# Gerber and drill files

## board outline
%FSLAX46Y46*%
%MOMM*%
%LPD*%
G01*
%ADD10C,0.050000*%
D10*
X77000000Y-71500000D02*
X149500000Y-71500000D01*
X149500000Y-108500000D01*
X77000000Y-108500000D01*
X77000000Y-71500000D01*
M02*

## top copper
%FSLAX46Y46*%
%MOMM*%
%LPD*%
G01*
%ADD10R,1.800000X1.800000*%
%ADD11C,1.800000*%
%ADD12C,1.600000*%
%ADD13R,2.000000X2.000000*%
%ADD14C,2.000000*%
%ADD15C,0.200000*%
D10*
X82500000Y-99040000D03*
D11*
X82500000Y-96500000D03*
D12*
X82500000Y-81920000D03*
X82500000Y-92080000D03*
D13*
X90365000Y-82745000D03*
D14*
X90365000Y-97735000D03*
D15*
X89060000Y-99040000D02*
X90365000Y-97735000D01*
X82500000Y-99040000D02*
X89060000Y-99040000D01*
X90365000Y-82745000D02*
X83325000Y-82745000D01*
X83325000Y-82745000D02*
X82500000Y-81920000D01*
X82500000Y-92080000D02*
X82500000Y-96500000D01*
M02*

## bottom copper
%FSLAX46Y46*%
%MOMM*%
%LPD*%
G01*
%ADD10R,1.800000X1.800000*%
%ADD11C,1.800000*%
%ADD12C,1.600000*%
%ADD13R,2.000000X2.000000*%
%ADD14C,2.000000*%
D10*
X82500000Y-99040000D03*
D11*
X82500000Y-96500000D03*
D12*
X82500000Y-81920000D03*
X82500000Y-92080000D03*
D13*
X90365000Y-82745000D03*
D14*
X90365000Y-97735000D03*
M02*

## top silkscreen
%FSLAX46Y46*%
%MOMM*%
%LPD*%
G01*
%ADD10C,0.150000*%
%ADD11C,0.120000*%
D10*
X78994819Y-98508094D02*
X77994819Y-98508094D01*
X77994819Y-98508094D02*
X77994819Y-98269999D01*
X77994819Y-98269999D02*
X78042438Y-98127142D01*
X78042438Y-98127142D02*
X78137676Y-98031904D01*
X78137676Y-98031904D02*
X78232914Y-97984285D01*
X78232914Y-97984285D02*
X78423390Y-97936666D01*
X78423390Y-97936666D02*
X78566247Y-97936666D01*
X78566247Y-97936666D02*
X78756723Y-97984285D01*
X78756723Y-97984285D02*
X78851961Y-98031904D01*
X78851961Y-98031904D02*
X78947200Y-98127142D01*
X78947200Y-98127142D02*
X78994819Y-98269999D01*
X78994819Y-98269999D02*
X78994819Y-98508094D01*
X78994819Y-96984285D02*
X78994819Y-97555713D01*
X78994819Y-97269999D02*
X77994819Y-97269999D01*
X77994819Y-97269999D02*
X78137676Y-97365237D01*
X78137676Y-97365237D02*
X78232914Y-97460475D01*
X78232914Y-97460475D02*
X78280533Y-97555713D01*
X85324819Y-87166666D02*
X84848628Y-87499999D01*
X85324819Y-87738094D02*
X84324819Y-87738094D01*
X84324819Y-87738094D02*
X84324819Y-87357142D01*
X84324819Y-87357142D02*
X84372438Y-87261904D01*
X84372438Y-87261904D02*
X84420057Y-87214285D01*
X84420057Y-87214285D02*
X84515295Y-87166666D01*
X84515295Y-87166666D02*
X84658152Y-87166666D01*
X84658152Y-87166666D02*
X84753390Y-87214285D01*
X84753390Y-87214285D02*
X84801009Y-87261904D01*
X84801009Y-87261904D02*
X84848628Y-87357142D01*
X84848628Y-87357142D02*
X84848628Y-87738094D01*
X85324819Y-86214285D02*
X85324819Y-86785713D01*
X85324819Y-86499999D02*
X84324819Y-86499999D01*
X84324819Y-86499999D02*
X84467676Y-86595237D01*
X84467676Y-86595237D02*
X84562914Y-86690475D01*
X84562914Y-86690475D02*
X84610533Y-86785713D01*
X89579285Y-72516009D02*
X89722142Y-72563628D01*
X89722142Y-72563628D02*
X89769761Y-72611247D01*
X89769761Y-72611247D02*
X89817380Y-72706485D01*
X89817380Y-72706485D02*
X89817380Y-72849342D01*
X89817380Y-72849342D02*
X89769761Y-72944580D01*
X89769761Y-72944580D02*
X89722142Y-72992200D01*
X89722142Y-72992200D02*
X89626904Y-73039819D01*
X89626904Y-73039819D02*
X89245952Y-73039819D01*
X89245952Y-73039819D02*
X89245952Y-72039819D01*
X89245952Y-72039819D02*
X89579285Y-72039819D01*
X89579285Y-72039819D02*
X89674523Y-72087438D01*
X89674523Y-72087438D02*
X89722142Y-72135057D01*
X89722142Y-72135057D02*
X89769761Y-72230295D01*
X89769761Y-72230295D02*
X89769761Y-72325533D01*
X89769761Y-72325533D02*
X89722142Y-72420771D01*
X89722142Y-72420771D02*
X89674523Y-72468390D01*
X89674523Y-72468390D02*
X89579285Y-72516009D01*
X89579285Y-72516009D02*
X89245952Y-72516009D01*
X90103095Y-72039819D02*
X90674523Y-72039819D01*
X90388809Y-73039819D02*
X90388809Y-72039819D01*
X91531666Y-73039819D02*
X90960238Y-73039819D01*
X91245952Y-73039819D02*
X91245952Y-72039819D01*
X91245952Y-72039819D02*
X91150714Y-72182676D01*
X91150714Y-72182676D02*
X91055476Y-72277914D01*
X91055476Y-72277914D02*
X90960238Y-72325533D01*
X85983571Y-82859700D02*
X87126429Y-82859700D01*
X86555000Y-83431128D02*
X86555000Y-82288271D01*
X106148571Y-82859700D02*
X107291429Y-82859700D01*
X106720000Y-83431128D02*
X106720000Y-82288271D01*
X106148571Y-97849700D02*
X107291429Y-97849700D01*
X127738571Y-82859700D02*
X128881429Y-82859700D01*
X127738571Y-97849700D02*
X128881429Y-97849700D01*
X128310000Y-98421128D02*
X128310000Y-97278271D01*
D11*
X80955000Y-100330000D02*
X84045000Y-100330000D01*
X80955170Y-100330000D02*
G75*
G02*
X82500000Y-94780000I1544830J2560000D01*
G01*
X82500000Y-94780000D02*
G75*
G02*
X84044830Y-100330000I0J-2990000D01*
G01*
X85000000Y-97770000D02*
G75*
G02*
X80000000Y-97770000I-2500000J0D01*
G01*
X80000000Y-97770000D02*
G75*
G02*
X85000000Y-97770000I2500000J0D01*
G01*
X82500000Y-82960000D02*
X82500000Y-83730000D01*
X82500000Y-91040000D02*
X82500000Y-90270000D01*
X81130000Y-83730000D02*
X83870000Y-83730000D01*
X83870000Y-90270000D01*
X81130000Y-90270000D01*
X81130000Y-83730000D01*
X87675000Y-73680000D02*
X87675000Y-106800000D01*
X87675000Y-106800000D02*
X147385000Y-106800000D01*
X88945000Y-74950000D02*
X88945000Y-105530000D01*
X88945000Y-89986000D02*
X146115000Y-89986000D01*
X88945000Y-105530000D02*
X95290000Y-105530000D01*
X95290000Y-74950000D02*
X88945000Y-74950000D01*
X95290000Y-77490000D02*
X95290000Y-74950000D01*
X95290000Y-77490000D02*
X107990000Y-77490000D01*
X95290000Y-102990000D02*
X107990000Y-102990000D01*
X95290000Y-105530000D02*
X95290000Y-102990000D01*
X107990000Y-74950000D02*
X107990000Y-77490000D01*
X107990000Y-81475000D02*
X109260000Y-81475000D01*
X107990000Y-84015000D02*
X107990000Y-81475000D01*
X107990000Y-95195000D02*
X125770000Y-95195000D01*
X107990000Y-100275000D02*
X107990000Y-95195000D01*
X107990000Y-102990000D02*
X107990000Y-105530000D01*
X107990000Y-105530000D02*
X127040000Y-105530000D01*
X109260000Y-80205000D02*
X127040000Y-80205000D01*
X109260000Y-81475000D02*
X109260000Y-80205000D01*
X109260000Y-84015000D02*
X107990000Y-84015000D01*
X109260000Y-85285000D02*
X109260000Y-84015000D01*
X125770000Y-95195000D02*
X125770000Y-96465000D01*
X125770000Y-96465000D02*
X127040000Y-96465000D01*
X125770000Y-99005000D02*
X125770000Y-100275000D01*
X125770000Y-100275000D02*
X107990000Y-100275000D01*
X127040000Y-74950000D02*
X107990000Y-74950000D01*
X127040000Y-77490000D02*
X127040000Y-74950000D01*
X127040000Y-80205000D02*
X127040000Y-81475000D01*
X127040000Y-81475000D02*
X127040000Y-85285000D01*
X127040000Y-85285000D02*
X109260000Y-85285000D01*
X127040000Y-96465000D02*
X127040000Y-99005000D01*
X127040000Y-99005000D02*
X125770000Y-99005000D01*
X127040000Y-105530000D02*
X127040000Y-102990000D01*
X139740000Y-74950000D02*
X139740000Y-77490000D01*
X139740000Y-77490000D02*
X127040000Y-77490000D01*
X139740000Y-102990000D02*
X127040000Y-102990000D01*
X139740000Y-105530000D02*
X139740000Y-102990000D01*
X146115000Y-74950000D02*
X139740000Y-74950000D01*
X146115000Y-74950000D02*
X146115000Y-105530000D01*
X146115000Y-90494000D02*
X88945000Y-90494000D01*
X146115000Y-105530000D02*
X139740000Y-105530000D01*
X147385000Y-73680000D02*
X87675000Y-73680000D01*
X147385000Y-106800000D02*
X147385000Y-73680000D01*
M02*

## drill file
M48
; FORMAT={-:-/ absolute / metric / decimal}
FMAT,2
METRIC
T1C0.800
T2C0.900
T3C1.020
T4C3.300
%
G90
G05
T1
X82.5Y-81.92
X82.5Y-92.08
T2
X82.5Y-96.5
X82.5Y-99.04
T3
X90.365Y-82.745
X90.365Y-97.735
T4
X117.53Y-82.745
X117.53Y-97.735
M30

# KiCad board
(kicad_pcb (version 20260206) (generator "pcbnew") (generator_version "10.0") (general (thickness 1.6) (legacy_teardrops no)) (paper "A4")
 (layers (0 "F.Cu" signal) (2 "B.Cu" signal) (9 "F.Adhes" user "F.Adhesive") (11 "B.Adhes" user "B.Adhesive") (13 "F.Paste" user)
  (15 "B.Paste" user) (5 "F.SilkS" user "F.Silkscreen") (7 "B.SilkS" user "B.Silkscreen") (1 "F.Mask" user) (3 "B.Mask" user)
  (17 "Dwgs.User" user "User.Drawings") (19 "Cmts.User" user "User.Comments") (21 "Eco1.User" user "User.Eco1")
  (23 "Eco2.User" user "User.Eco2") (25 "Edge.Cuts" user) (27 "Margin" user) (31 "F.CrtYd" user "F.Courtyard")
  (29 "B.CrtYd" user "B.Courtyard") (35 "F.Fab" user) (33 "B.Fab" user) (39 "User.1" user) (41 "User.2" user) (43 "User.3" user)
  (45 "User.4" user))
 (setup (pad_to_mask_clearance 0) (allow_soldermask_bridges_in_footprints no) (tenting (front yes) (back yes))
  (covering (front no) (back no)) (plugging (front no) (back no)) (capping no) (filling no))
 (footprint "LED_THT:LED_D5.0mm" (layer "F.Cu") (at 82.5 99.04 90)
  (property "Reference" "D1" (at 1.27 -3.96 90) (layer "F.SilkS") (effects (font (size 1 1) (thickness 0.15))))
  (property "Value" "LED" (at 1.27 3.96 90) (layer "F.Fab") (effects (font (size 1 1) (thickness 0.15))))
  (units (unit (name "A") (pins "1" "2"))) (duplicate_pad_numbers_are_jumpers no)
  (fp_line (start -1.29 -1.545) (end -1.29 1.545) (stroke (width 0.12) (type solid)) (layer "F.SilkS"))
  (fp_arc (start -1.29 -1.54483) (mid 2.071779 -2.880495) (end 4.26 0) (stroke (width 0.12) (type solid)) (layer "F.SilkS"))
  (fp_arc (start 4.26 0) (mid 2.071779 2.880495) (end -1.29 1.54483) (stroke (width 0.12) (type solid)) (layer "F.SilkS"))
  (fp_circle (center 1.27 0) (end 3.77 0) (stroke (width 0.12) (type solid)) (fill no) (layer "F.SilkS"))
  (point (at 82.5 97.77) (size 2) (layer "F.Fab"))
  (pad "1" thru_hole rect (at 0 0 90) (size 1.8 1.8) (drill 0.9) (layers "*.Cu" "*.Mask") (remove_unused_layers no) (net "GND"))
  (pad "2" thru_hole circle (at 2.54 0 90) (size 1.8 1.8) (drill 0.9) (layers "*.Cu" "*.Mask") (remove_unused_layers no) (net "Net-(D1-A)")))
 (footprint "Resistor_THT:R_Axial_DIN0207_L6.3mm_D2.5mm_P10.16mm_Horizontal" (layer "F.Cu") (at 82.5 81.92 -90)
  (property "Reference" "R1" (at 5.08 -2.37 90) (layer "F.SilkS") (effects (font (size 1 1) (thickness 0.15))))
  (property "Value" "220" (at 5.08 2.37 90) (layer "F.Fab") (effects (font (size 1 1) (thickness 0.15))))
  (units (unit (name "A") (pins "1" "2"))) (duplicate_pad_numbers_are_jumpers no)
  (fp_line (start 1.04 0) (end 1.81 0) (stroke (width 0.12) (type solid)) (layer "F.SilkS"))
  (fp_line (start 9.12 0) (end 8.35 0) (stroke (width 0.12) (type solid)) (layer "F.SilkS"))
  (fp_rect (start 1.81 -1.37) (end 8.35 1.37) (stroke (width 0.12) (type solid)) (fill no) (layer "F.SilkS"))
  (pad "1" thru_hole circle (at 0 0 270) (size 1.6 1.6) (drill 0.8) (layers "*.Cu" "*.Mask") (remove_unused_layers no) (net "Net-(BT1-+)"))
  (pad "2" thru_hole circle (at 10.16 0 270) (size 1.6 1.6) (drill 0.8) (layers "*.Cu" "*.Mask") (remove_unused_layers no)
   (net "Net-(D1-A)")))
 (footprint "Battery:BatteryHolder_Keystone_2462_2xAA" (layer "F.Cu") (at 90.365 82.745)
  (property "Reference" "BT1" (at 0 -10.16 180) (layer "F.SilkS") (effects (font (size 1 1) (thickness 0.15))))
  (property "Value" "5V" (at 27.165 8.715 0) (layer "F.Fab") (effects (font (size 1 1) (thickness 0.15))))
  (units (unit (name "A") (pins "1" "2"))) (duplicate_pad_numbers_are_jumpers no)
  (fp_line (start -2.69 -9.065) (end -2.69 24.055) (stroke (width 0.12) (type solid)) (layer "F.SilkS"))
  (fp_line (start -2.69 24.055) (end 57.02 24.055) (stroke (width 0.12) (type solid)) (layer "F.SilkS"))
  (fp_line (start -1.42 -7.795) (end -1.42 22.785) (stroke (width 0.12) (type solid)) (layer "F.SilkS"))
  (fp_line (start -1.42 7.241) (end 55.75 7.241) (stroke (width 0.12) (type solid)) (layer "F.SilkS"))
  (fp_line (start -1.42 22.785) (end 4.925 22.785) (stroke (width 0.12) (type solid)) (layer "F.SilkS"))
  (fp_line (start 4.925 -7.795) (end -1.42 -7.795) (stroke (width 0.12) (type solid)) (layer "F.SilkS"))
  (fp_line (start 4.925 -5.255) (end 4.925 -7.795) (stroke (width 0.12) (type solid)) (layer "F.SilkS"))
  (fp_line (start 4.925 -5.255) (end 17.625 -5.255) (stroke (width 0.12) (type solid)) (layer "F.SilkS"))
  (fp_line (start 4.925 20.245) (end 17.625 20.245) (stroke (width 0.12) (type solid)) (layer "F.SilkS"))
  (fp_line (start 4.925 22.785) (end 4.925 20.245) (stroke (width 0.12) (type solid)) (layer "F.SilkS"))
  (fp_line (start 17.625 -7.795) (end 17.625 -5.255) (stroke (width 0.12) (type solid)) (layer "F.SilkS"))
  (fp_line (start 17.625 -1.27) (end 18.895 -1.27) (stroke (width 0.12) (type solid)) (layer "F.SilkS"))
  (fp_line (start 17.625 1.27) (end 17.625 -1.27) (stroke (width 0.12) (type solid)) (layer "F.SilkS"))
  (fp_line (start 17.625 12.45) (end 35.405 12.45) (stroke (width 0.12) (type solid)) (layer "F.SilkS"))
  (fp_line (start 17.625 17.53) (end 17.625 12.45) (stroke (width 0.12) (type solid)) (layer "F.SilkS"))
  (fp_line (start 17.625 20.245) (end 17.625 22.785) (stroke (width 0.12) (type solid)) (layer "F.SilkS"))
  (fp_line (start 17.625 22.785) (end 36.675 22.785) (stroke (width 0.12) (type solid)) (layer "F.SilkS"))
  (fp_line (start 18.895 -2.54) (end 36.675 -2.54) (stroke (width 0.12) (type solid)) (layer "F.SilkS"))
  (fp_line (start 18.895 -1.27) (end 18.895 -2.54) (stroke (width 0.12) (type solid)) (layer "F.SilkS"))
  (fp_line (start 18.895 1.27) (end 17.625 1.27) (stroke (width 0.12) (type solid)) (layer "F.SilkS"))
  (fp_line (start 18.895 2.54) (end 18.895 1.27) (stroke (width 0.12) (type solid)) (layer "F.SilkS"))
  (fp_line (start 35.405 12.45) (end 35.405 13.72) (stroke (width 0.12) (type solid)) (layer "F.SilkS"))
  (fp_line (start 35.405 13.72) (end 36.675 13.72) (stroke (width 0.12) (type solid)) (layer "F.SilkS"))
  (fp_line (start 35.405 16.26) (end 35.405 17.53) (stroke (width 0.12) (type solid)) (layer "F.SilkS"))
  (fp_line (start 35.405 17.53) (end 17.625 17.53) (stroke (width 0.12) (type solid)) (layer "F.SilkS"))
  (fp_line (start 36.675 -7.795) (end 17.625 -7.795) (stroke (width 0.12) (type solid)) (layer "F.SilkS"))
  (fp_line (start 36.675 -5.255) (end 36.675 -7.795) (stroke (width 0.12) (type solid)) (layer "F.SilkS"))
  (fp_line (start 36.675 -2.54) (end 36.675 -1.27) (stroke (width 0.12) (type solid)) (layer "F.SilkS"))
  (fp_line (start 36.675 -1.27) (end 36.675 2.54) (stroke (width 0.12) (type solid)) (layer "F.SilkS"))
  (fp_line (start 36.675 2.54) (end 18.895 2.54) (stroke (width 0.12) (type solid)) (layer "F.SilkS"))
  (fp_line (start 36.675 13.72) (end 36.675 16.26) (stroke (width 0.12) (type solid)) (layer "F.SilkS"))
  (fp_line (start 36.675 16.26) (end 35.405 16.26) (stroke (width 0.12) (type solid)) (layer "F.SilkS"))
  (fp_line (start 36.675 22.785) (end 36.675 20.245) (stroke (width 0.12) (type solid)) (layer "F.SilkS"))
  (fp_line (start 49.375 -7.795) (end 49.375 -5.255) (stroke (width 0.12) (type solid)) (layer "F.SilkS"))
  (fp_line (start 49.375 -5.255) (end 36.675 -5.255) (stroke (width 0.12) (type solid)) (layer "F.SilkS"))
  (fp_line (start 49.375 20.245) (end 36.675 20.245) (stroke (width 0.12) (type solid)) (layer "F.SilkS"))
  (fp_line (start 49.375 22.785) (end 49.375 20.245) (stroke (width 0.12) (type solid)) (layer "F.SilkS"))
  (fp_line (start 55.75 -7.795) (end 49.375 -7.795) (stroke (width 0.12) (type solid)) (layer "F.SilkS"))
  (fp_line (start 55.75 -7.795) (end 55.75 22.785) (stroke (width 0.12) (type solid)) (layer "F.SilkS"))
  (fp_line (start 55.75 7.749) (end -1.42 7.749) (stroke (width 0.12) (type solid)) (layer "F.SilkS"))
  (fp_line (start 55.75 22.785) (end 49.375 22.785) (stroke (width 0.12) (type solid)) (layer "F.SilkS"))
  (fp_line (start 57.02 -9.065) (end -2.69 -9.065) (stroke (width 0.12) (type solid)) (layer "F.SilkS"))
  (fp_line (start 57.02 24.055) (end 57.02 -9.065) (stroke (width 0.12) (type solid)) (layer "F.SilkS"))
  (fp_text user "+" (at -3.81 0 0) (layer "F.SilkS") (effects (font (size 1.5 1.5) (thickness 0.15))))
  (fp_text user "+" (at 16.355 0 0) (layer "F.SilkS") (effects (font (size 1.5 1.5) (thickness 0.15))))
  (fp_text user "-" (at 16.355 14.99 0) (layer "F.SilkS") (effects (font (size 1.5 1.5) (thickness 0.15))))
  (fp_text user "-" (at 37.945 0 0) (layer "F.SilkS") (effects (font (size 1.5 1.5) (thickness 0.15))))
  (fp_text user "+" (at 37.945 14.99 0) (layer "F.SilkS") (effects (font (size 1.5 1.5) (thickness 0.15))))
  (pad "" np_thru_hole circle (at 27.165 0) (size 3.3 3.3) (drill 3.3) (layers "*.Cu" "*.Mask"))
  (pad "" np_thru_hole circle (at 27.165 14.99) (size 3.3 3.3) (drill 3.3) (layers "*.Cu" "*.Mask"))
  (pad "1" thru_hole rect (at 0 0) (size 2 2) (drill 1.02) (layers "*.Cu" "*.Mask") (remove_unused_layers no) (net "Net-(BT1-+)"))
  (pad "2" thru_hole circle (at 0 14.99) (size 2 2) (drill 1.02) (layers "*.Cu" "*.Mask") (remove_unused_layers no) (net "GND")))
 (gr_rect (start 77 71.5) (end 149.5 108.5) (stroke (width 0.05) (type default)) (fill no) (layer "Edge.Cuts"))
 (segment (start 89.06 99.04) (end 90.365 97.735) (width 0.2) (layer "F.Cu") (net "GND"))
 (segment (start 82.5 99.04) (end 89.06 99.04) (width 0.2) (layer "F.Cu") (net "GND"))
 (segment (start 90.365 82.745) (end 83.325 82.745) (width 0.2) (layer "F.Cu") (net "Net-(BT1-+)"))
 (segment (start 83.325 82.745) (end 82.5 81.92) (width 0.2) (layer "F.Cu") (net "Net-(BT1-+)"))
 (segment (start 82.5 92.08) (end 82.5 96.5) (width 0.2) (layer "F.Cu") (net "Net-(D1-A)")))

